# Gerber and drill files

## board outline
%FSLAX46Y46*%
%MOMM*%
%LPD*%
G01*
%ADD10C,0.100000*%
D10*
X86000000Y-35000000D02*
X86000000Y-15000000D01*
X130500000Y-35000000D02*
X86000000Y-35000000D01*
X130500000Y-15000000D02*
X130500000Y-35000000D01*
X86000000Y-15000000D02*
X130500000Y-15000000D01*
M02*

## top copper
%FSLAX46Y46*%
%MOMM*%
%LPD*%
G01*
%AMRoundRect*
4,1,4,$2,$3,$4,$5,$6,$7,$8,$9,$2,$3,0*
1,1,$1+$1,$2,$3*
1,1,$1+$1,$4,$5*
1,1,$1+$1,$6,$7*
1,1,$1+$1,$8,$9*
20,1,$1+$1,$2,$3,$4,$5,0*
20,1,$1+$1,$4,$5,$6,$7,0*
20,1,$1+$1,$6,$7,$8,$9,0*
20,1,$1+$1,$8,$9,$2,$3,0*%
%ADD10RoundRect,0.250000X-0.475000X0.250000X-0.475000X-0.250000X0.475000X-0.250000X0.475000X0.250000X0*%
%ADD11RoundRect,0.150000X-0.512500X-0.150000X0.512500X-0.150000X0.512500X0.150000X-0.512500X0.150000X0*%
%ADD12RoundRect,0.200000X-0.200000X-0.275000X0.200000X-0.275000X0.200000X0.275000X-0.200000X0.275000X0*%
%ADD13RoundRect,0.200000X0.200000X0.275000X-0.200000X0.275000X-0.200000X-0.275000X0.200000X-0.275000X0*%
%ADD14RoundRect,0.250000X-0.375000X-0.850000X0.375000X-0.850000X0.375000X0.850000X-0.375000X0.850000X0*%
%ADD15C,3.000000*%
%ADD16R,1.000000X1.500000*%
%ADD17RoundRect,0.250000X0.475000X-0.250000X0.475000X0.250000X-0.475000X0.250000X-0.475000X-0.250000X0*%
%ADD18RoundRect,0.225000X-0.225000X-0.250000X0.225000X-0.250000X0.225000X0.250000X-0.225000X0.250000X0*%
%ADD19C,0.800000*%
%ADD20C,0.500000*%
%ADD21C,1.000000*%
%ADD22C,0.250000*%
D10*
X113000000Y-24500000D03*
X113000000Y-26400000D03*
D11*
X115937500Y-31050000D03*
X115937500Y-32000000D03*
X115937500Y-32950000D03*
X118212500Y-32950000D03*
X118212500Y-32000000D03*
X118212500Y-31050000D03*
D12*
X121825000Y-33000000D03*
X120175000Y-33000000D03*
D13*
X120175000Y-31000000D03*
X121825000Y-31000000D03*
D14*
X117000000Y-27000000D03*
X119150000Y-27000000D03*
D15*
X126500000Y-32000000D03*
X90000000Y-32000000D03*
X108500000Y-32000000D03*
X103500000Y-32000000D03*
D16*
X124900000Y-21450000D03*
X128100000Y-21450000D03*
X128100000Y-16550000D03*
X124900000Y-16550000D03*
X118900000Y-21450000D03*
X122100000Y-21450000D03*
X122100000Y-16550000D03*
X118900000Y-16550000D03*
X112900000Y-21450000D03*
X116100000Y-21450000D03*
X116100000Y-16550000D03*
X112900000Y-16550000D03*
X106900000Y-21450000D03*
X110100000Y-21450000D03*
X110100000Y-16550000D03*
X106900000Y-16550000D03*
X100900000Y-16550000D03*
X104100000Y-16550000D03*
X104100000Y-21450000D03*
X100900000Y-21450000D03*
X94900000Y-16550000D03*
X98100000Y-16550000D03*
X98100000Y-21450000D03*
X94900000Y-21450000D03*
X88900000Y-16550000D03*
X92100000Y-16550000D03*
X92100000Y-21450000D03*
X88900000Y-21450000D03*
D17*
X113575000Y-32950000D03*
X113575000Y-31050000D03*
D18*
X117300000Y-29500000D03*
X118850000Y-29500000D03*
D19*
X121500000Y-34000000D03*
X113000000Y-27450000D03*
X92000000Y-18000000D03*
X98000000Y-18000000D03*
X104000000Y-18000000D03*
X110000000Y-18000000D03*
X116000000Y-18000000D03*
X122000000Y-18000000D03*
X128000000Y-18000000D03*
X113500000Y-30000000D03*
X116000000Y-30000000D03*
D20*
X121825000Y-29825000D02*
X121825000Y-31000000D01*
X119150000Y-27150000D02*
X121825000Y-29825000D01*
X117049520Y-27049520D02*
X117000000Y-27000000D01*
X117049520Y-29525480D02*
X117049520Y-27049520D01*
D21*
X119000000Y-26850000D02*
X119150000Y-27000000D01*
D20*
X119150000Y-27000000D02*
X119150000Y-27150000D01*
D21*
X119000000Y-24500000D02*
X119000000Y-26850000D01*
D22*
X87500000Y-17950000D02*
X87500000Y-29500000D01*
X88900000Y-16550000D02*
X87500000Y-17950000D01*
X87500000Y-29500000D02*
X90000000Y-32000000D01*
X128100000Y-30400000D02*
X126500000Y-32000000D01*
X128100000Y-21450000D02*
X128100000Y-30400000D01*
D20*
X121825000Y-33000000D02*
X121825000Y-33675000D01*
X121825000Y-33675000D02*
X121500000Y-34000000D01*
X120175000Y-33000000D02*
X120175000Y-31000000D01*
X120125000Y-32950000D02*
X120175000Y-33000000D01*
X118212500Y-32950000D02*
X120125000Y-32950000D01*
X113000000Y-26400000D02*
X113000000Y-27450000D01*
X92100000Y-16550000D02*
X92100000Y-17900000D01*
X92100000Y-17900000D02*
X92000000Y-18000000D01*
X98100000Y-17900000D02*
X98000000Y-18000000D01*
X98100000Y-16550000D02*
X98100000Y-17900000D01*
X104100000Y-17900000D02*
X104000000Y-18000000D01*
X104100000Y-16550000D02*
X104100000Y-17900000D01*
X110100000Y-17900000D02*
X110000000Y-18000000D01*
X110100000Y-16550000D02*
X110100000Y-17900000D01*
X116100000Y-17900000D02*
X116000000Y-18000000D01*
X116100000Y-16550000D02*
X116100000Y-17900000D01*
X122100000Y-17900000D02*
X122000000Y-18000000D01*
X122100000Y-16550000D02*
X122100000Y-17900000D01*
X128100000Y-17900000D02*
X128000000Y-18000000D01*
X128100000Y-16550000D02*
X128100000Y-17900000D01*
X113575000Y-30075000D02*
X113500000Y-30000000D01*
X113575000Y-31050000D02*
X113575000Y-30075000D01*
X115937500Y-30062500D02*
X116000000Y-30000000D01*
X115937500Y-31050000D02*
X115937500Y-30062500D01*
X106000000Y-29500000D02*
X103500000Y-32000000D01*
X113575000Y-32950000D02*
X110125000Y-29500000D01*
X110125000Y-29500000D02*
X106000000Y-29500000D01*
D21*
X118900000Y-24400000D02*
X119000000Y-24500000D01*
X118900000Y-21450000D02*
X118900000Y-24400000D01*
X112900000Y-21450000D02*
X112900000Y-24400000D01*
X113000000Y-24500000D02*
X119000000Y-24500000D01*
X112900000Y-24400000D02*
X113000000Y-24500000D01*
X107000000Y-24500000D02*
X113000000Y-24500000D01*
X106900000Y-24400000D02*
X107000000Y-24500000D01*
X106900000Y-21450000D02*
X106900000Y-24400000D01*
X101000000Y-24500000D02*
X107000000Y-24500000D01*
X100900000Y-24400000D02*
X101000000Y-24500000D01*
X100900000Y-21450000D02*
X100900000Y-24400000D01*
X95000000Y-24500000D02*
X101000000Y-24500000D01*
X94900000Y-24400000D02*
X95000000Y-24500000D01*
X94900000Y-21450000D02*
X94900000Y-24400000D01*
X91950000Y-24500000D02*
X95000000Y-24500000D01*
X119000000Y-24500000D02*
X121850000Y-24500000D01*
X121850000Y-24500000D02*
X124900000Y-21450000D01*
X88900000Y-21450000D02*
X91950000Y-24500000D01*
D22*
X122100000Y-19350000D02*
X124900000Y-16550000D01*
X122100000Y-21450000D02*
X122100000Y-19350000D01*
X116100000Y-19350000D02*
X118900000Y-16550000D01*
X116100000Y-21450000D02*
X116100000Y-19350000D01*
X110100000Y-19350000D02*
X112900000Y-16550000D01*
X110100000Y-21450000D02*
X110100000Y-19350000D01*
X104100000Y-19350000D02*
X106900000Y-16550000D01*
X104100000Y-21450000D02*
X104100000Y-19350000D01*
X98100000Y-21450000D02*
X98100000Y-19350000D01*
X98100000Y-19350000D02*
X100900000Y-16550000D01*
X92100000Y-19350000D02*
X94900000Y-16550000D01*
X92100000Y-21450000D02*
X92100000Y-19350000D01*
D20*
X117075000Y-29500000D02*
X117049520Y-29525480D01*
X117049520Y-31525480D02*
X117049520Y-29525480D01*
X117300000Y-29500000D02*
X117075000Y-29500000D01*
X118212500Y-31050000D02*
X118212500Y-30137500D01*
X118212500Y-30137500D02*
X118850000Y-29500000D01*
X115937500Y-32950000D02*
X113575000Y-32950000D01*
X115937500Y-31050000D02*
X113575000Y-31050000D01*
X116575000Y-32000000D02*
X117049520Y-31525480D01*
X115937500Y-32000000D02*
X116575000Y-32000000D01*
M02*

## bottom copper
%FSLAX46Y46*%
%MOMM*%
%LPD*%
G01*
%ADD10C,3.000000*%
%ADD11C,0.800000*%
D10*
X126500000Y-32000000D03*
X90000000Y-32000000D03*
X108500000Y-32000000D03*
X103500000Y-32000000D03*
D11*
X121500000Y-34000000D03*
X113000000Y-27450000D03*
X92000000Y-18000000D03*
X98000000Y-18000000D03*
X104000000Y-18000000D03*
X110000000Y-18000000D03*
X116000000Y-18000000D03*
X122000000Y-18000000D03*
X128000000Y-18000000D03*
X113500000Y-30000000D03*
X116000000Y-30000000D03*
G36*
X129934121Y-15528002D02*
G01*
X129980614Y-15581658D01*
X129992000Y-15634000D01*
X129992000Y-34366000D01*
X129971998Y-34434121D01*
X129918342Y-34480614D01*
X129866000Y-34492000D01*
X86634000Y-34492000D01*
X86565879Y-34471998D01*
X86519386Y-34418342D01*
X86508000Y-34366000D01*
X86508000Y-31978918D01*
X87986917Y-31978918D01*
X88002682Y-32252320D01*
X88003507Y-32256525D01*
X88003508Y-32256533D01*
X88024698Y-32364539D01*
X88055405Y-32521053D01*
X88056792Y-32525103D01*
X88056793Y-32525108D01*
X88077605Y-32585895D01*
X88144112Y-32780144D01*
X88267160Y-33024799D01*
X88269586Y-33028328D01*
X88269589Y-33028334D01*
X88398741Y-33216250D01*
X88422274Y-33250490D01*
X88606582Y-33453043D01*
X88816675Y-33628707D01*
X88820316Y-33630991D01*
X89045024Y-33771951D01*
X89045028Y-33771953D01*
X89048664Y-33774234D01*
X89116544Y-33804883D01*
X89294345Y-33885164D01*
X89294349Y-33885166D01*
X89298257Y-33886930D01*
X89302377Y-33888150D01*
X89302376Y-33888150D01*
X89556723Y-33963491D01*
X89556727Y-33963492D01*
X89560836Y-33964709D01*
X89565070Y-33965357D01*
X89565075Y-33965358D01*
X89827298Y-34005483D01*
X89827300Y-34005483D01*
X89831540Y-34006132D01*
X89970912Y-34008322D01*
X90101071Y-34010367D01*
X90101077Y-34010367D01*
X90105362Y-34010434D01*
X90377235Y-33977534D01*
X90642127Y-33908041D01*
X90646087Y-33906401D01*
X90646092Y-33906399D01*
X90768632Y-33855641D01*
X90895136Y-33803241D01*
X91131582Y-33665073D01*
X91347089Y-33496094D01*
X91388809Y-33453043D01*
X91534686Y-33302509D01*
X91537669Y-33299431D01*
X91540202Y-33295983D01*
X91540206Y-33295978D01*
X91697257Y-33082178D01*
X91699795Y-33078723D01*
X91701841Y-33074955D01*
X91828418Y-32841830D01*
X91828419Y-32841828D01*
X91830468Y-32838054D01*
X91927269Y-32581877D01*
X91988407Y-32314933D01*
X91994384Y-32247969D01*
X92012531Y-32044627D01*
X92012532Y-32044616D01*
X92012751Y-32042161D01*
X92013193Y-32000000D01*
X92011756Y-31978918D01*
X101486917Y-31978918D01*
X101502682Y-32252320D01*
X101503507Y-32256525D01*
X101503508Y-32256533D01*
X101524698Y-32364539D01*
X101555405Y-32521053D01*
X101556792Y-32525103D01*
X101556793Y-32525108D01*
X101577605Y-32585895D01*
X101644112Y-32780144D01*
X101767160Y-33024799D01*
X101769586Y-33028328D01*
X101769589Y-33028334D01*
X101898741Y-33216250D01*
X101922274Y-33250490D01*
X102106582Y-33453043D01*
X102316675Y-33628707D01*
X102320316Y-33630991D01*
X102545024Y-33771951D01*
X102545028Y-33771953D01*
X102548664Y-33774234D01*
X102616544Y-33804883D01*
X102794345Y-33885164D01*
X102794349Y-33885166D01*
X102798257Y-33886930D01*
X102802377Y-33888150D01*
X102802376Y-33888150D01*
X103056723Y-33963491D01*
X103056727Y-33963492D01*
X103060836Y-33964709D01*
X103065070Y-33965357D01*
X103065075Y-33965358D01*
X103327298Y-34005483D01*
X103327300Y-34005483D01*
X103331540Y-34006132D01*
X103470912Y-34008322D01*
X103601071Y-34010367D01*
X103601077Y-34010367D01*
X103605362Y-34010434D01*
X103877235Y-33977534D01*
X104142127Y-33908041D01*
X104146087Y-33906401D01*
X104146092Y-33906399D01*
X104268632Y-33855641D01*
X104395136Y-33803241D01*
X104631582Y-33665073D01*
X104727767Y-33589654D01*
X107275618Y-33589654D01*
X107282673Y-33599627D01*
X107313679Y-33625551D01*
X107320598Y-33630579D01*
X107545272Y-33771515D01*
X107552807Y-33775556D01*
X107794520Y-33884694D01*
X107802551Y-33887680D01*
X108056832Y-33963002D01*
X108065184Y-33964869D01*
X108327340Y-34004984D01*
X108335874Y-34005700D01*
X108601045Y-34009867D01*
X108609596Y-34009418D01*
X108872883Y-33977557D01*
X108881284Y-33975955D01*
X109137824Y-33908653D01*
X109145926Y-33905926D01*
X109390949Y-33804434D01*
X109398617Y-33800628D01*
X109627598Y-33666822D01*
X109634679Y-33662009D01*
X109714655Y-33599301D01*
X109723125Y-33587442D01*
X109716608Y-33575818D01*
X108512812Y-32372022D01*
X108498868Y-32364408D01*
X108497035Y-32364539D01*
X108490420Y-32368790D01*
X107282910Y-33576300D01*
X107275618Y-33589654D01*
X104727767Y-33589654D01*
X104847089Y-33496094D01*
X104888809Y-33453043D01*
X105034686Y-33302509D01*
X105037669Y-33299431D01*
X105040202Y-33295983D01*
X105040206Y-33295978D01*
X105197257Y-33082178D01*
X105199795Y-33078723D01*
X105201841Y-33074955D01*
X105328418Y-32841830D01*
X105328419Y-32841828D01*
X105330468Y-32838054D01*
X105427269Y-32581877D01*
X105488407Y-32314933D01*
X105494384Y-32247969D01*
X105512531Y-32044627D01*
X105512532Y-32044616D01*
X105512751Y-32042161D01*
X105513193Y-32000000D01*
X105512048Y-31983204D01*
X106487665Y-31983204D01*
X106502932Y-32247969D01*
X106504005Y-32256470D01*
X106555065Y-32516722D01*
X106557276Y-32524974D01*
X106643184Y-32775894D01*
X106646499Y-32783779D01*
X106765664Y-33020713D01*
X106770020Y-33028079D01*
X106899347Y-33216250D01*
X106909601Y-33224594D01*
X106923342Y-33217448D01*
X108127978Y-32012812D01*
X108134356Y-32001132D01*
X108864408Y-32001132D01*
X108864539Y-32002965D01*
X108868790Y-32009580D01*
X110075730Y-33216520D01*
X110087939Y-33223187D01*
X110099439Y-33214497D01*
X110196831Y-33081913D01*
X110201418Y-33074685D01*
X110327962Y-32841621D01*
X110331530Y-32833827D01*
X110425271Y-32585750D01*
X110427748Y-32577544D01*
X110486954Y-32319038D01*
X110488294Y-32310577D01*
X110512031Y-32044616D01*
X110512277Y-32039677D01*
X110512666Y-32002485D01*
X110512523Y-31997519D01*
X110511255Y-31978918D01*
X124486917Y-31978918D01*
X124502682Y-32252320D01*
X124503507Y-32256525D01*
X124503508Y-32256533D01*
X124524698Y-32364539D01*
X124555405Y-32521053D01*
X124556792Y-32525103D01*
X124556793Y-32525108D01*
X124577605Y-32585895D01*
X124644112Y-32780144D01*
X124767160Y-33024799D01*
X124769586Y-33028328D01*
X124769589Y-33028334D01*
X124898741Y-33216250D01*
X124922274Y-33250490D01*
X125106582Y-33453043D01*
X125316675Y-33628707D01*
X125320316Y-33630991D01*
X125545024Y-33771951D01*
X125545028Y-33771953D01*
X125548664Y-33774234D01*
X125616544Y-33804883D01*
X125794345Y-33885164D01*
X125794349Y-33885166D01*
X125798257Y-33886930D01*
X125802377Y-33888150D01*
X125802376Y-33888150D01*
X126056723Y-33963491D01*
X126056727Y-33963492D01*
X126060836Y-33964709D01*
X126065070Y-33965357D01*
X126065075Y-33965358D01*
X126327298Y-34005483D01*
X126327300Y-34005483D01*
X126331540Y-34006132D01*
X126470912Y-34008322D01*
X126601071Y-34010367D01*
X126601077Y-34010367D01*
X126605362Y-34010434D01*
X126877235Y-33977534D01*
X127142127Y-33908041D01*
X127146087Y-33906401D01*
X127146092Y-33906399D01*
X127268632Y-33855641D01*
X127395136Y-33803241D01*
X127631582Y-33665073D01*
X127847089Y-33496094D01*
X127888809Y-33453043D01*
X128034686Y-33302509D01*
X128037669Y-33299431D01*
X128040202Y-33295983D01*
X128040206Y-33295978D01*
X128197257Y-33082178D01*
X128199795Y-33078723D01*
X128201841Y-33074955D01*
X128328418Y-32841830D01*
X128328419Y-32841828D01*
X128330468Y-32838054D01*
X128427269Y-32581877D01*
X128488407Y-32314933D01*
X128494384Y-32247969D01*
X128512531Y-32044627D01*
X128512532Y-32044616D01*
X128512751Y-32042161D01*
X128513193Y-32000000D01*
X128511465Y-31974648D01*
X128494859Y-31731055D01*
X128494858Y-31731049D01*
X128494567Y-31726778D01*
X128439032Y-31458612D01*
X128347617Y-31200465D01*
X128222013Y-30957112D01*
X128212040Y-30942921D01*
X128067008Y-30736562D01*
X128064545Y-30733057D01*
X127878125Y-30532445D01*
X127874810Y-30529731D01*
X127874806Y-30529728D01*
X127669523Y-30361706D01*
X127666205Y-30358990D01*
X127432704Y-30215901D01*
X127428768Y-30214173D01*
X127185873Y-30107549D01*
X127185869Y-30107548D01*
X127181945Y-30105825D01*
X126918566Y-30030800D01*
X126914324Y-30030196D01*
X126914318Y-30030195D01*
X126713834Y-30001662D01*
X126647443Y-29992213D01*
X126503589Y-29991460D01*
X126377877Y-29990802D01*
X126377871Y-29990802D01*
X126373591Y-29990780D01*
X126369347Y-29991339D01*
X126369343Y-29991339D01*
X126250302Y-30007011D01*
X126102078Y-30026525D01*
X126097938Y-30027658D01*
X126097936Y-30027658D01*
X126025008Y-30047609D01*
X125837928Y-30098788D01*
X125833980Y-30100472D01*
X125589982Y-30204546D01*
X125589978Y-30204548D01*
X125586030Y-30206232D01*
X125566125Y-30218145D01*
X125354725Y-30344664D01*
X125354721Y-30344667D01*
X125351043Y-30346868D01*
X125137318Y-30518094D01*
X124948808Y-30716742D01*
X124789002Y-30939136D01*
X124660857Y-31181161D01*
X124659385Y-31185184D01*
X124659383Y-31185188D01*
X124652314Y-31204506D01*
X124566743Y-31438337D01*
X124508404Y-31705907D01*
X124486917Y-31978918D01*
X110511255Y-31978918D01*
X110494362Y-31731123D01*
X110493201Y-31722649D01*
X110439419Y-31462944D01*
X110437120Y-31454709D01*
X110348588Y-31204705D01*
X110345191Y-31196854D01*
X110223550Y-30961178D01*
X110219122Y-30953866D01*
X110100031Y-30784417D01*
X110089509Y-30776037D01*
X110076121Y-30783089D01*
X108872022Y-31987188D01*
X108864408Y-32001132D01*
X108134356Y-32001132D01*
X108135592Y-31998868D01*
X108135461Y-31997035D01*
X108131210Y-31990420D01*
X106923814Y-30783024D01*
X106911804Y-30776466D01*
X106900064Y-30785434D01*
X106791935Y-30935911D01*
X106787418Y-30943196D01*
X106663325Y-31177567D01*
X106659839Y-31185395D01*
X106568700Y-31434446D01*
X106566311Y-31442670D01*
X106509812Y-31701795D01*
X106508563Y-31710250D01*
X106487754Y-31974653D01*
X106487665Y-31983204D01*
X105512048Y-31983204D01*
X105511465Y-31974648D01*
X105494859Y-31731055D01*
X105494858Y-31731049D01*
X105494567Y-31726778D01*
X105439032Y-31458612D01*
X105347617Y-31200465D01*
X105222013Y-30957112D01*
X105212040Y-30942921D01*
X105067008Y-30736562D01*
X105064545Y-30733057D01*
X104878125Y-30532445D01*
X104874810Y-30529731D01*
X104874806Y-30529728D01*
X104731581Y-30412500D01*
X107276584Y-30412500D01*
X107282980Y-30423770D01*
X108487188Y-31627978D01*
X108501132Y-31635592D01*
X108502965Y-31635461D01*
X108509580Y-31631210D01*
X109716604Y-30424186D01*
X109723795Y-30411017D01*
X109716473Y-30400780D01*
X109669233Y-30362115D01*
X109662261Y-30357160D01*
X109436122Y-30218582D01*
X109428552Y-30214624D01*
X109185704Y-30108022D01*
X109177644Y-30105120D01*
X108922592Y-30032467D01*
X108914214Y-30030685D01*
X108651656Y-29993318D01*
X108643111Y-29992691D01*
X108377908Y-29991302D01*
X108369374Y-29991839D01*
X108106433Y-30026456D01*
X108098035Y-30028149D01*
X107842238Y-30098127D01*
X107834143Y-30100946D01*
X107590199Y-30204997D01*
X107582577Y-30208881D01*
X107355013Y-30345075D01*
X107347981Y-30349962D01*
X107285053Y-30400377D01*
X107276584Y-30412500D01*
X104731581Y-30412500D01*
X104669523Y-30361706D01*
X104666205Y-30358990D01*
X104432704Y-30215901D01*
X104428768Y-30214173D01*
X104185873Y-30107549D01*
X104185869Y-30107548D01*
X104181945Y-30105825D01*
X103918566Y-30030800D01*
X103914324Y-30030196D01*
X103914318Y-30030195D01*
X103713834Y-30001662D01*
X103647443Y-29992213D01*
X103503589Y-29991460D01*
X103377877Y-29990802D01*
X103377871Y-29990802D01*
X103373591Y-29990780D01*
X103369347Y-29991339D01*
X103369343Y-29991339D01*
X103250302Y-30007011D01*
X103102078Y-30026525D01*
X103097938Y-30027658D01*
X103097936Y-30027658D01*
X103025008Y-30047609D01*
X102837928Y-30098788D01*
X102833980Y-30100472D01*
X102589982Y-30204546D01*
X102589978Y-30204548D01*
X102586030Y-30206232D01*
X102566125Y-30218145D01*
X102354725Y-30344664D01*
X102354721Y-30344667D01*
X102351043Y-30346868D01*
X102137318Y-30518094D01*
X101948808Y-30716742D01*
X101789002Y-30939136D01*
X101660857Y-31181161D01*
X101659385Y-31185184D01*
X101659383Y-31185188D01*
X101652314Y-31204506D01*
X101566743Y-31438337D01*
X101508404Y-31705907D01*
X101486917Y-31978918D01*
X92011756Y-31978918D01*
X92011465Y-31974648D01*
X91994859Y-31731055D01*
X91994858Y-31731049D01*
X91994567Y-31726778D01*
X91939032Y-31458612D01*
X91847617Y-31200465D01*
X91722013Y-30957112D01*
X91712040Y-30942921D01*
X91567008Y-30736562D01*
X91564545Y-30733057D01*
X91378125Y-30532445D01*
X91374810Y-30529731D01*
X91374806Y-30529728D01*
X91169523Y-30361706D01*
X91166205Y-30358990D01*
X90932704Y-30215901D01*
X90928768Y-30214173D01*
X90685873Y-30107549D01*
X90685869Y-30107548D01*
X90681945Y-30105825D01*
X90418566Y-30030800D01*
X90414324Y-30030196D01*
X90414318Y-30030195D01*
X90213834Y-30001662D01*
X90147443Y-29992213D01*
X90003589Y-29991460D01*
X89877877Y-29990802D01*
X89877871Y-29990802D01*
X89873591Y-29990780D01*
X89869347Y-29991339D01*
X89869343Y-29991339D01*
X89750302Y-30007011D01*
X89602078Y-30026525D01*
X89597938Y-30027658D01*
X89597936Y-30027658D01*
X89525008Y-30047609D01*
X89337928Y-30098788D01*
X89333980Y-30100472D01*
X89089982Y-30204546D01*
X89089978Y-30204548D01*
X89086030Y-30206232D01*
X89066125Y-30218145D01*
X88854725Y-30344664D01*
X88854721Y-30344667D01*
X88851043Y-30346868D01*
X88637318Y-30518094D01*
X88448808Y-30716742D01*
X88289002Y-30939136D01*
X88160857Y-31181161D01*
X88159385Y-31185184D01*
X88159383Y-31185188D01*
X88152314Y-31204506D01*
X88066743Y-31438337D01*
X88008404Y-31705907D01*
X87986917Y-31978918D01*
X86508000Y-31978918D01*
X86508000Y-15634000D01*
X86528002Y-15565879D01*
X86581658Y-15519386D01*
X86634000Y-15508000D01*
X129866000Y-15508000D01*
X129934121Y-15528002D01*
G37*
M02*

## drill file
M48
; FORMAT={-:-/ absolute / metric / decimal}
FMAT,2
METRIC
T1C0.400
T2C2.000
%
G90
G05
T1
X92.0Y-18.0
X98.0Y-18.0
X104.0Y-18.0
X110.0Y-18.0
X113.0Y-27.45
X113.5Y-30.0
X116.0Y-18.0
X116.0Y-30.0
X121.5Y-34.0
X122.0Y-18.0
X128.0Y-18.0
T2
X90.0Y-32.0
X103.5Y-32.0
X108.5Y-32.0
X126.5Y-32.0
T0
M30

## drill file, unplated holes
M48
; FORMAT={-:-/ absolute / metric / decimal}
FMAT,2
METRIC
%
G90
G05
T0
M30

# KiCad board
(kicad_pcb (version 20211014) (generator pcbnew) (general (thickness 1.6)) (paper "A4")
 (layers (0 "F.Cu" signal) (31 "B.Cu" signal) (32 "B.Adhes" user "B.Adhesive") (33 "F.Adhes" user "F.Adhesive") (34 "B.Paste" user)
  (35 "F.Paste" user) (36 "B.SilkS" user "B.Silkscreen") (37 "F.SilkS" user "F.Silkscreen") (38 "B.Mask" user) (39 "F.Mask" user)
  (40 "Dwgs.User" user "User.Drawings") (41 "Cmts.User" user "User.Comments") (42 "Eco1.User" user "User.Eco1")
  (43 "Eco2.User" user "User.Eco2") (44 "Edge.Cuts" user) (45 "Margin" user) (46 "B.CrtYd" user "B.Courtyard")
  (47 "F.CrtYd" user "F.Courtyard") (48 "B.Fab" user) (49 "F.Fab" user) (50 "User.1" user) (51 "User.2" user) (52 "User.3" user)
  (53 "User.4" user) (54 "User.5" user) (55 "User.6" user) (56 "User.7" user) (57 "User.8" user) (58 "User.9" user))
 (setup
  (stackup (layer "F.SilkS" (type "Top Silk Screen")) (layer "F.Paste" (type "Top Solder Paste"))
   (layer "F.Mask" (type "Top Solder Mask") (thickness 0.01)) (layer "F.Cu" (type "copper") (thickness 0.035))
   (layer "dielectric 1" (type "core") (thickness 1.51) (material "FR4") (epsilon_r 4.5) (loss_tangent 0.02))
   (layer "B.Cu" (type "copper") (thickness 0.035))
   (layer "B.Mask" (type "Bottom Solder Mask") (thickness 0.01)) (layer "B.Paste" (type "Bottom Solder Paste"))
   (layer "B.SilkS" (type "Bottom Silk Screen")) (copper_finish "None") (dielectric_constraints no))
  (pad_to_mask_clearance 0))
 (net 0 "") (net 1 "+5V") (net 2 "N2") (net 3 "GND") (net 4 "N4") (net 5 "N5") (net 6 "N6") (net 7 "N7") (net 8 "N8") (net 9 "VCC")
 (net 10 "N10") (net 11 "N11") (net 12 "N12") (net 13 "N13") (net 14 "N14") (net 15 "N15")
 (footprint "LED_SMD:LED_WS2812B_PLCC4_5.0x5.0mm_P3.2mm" (layer "F.Cu") (at 114.5 19 90)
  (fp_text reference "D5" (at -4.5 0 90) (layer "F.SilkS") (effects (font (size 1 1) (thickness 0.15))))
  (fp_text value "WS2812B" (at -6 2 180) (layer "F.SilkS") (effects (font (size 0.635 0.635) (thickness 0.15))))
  (pad "1" smd rect (at -2.45 -1.6 90) (size 1.5 1) (layers "F.Cu" "F.Paste" "F.Mask") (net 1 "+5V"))
  (pad "2" smd rect (at -2.45 1.6 90) (size 1.5 1) (layers "F.Cu" "F.Paste" "F.Mask") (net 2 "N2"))
  (pad "3" smd rect (at 2.45 1.6 90) (size 1.5 1) (layers "F.Cu" "F.Paste" "F.Mask") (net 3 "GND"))
  (pad "4" smd rect (at 2.45 -1.6 90) (size 1.5 1) (layers "F.Cu" "F.Paste" "F.Mask") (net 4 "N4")))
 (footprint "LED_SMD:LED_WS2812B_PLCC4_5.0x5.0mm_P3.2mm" (layer "F.Cu") (at 90.5 19 90)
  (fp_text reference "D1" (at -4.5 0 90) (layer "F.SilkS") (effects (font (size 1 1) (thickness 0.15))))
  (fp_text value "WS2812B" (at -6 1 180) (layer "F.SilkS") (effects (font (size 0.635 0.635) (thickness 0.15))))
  (pad "1" smd rect (at -2.45 -1.6 90) (size 1.5 1) (layers "F.Cu" "F.Paste" "F.Mask") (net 1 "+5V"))
  (pad "2" smd rect (at -2.45 1.6 90) (size 1.5 1) (layers "F.Cu" "F.Paste" "F.Mask") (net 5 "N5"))
  (pad "3" smd rect (at 2.45 1.6 90) (size 1.5 1) (layers "F.Cu" "F.Paste" "F.Mask") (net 3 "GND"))
  (pad "4" smd rect (at 2.45 -1.6 90) (size 1.5 1) (layers "F.Cu" "F.Paste" "F.Mask") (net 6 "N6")))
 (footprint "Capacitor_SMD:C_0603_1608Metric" (layer "F.Cu") (at 118.075 29.5)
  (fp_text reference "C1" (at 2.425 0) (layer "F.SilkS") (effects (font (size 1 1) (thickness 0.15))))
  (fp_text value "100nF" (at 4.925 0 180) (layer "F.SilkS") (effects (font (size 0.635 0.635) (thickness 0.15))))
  (pad "1" smd roundrect (at -0.775 0) (size 0.9 0.95) (layers "F.Cu" "F.Paste" "F.Mask") (roundrect_rratio 0.25) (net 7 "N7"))
  (pad "2" smd roundrect (at 0.775 0) (size 0.9 0.95) (layers "F.Cu" "F.Paste" "F.Mask") (roundrect_rratio 0.25) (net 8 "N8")))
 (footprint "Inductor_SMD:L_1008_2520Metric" (layer "F.Cu") (at 118.075 27)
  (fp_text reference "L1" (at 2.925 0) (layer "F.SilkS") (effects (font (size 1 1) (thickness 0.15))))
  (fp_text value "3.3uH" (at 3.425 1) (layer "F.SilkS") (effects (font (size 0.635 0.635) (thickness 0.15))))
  (pad "1" smd roundrect (at -1.075 0) (size 1.25 2.2) (layers "F.Cu" "F.Paste" "F.Mask") (roundrect_rratio 0.2) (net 7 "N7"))
  (pad "2" smd roundrect (at 1.075 0) (size 1.25 2.2) (layers "F.Cu" "F.Paste" "F.Mask") (roundrect_rratio 0.2) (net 1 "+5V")))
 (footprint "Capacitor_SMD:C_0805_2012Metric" (layer "F.Cu") (at 113 25.45 -90)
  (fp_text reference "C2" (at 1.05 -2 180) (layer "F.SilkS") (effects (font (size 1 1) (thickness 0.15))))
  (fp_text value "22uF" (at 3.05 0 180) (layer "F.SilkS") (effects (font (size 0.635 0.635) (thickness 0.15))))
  (pad "1" smd roundrect (at -0.95 0 270) (size 1 1.45) (layers "F.Cu" "F.Paste" "F.Mask") (roundrect_rratio 0.25) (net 1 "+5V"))
  (pad "2" smd roundrect (at 0.95 0 270) (size 1 1.45) (layers "F.Cu" "F.Paste" "F.Mask") (roundrect_rratio 0.25) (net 3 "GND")))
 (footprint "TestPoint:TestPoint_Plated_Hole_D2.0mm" (layer "F.Cu") (at 90 32)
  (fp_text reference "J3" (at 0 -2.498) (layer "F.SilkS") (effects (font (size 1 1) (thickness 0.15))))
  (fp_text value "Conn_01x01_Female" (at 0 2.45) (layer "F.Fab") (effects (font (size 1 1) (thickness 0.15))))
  (pad "1" thru_hole circle (at 0 0) (size 3 3) (drill 2) (layers *.Cu *.Mask) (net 6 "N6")))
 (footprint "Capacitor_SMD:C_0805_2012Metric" (layer "F.Cu") (at 113.575 32 90)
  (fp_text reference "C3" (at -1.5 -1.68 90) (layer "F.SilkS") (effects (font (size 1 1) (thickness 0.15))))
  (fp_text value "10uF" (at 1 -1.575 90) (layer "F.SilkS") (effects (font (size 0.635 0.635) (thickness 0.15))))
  (pad "1" smd roundrect (at -0.95 0 90) (size 1 1.45) (layers "F.Cu" "F.Paste" "F.Mask") (roundrect_rratio 0.25) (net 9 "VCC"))
  (pad "2" smd roundrect (at 0.95 0 90) (size 1 1.45) (layers "F.Cu" "F.Paste" "F.Mask") (roundrect_rratio 0.25) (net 3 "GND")))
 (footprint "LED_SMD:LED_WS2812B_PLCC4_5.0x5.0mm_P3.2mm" (layer "F.Cu") (at 120.5 19 90)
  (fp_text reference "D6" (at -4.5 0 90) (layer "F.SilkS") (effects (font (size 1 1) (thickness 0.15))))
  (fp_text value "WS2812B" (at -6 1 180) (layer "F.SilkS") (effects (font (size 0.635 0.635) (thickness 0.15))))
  (pad "1" smd rect (at -2.45 -1.6 90) (size 1.5 1) (layers "F.Cu" "F.Paste" "F.Mask") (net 1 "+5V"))
  (pad "2" smd rect (at -2.45 1.6 90) (size 1.5 1) (layers "F.Cu" "F.Paste" "F.Mask") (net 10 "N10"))
  (pad "3" smd rect (at 2.45 1.6 90) (size 1.5 1) (layers "F.Cu" "F.Paste" "F.Mask") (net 3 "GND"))
  (pad "4" smd rect (at 2.45 -1.6 90) (size 1.5 1) (layers "F.Cu" "F.Paste" "F.Mask") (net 2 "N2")))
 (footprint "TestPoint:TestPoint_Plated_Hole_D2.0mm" (layer "F.Cu") (at 103.5 32)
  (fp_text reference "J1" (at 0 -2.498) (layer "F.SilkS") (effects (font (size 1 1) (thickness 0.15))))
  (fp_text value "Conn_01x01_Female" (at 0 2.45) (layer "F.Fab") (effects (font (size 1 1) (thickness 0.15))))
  (pad "1" thru_hole circle (at 0 0) (size 3 3) (drill 2) (layers *.Cu *.Mask) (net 9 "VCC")))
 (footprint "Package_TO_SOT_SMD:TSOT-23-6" (layer "F.Cu") (at 117.075 32)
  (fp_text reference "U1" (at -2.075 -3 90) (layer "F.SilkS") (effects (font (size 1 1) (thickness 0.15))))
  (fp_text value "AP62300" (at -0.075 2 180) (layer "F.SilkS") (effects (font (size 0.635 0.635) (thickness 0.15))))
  (pad "1" smd roundrect (at -1.1375 -0.95) (size 1.325 0.6) (layers "F.Cu" "F.Paste" "F.Mask") (roundrect_rratio 0.25) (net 3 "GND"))
  (pad "2" smd roundrect (at -1.1375 0) (size 1.325 0.6) (layers "F.Cu" "F.Paste" "F.Mask") (roundrect_rratio 0.25) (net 7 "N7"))
  (pad "3" smd roundrect (at -1.1375 0.95) (size 1.325 0.6) (layers "F.Cu" "F.Paste" "F.Mask") (roundrect_rratio 0.25) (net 9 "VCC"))
  (pad "4" smd roundrect (at 1.1375 0.95) (size 1.325 0.6) (layers "F.Cu" "F.Paste" "F.Mask") (roundrect_rratio 0.25) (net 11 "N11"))
  (pad "5" smd roundrect (at 1.1375 0) (size 1.325 0.6) (layers "F.Cu" "F.Paste" "F.Mask") (roundrect_rratio 0.25) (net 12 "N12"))
  (pad "6" smd roundrect (at 1.1375 -0.95) (size 1.325 0.6) (layers "F.Cu" "F.Paste" "F.Mask") (roundrect_rratio 0.25) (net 8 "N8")))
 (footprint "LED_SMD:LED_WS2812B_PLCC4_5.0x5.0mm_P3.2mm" (layer "F.Cu") (at 102.5 19 90)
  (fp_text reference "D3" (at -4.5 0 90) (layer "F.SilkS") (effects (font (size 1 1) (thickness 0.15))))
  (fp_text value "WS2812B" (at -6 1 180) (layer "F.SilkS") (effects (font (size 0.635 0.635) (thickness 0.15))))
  (pad "1" smd rect (at -2.45 -1.6 90) (size 1.5 1) (layers "F.Cu" "F.Paste" "F.Mask") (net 1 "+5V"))
  (pad "2" smd rect (at -2.45 1.6 90) (size 1.5 1) (layers "F.Cu" "F.Paste" "F.Mask") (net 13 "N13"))
  (pad "3" smd rect (at 2.45 1.6 90) (size 1.5 1) (layers "F.Cu" "F.Paste" "F.Mask") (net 3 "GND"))
  (pad "4" smd rect (at 2.45 -1.6 90) (size 1.5 1) (layers "F.Cu" "F.Paste" "F.Mask") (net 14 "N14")))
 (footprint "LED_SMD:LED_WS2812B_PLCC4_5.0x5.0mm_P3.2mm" (layer "F.Cu") (at 126.5 19 90)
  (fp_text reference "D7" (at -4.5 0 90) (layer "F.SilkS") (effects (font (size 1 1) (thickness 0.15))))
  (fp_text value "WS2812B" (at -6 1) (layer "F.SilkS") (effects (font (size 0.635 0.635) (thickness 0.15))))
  (pad "1" smd rect (at -2.45 -1.6 90) (size 1.5 1) (layers "F.Cu" "F.Paste" "F.Mask") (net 1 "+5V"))
  (pad "2" smd rect (at -2.45 1.6 90) (size 1.5 1) (layers "F.Cu" "F.Paste" "F.Mask") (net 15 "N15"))
  (pad "3" smd rect (at 2.45 1.6 90) (size 1.5 1) (layers "F.Cu" "F.Paste" "F.Mask") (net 3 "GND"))
  (pad "4" smd rect (at 2.45 -1.6 90) (size 1.5 1) (layers "F.Cu" "F.Paste" "F.Mask") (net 10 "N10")))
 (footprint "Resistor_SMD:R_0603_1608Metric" (layer "F.Cu") (at 121 31 180)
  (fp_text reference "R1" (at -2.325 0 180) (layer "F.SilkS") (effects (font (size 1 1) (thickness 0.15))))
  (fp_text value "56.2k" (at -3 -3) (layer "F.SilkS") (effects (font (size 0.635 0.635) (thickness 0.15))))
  (pad "1" smd roundrect (at -0.825 0 180) (size 0.8 0.95) (layers "F.Cu" "F.Paste" "F.Mask") (roundrect_rratio 0.25) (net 1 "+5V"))
  (pad "2" smd roundrect (at 0.825 0 180) (size 0.8 0.95) (layers "F.Cu" "F.Paste" "F.Mask") (roundrect_rratio 0.25) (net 11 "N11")))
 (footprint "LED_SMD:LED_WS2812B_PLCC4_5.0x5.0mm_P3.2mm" (layer "F.Cu") (at 96.5 19 90)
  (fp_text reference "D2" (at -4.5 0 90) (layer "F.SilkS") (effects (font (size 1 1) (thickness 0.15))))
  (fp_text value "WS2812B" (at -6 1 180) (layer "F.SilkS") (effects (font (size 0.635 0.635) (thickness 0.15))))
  (pad "1" smd rect (at -2.45 -1.6 90) (size 1.5 1) (layers "F.Cu" "F.Paste" "F.Mask") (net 1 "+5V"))
  (pad "2" smd rect (at -2.45 1.6 90) (size 1.5 1) (layers "F.Cu" "F.Paste" "F.Mask") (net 14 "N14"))
  (pad "3" smd rect (at 2.45 1.6 90) (size 1.5 1) (layers "F.Cu" "F.Paste" "F.Mask") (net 3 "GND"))
  (pad "4" smd rect (at 2.45 -1.6 90) (size 1.5 1) (layers "F.Cu" "F.Paste" "F.Mask") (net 5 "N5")))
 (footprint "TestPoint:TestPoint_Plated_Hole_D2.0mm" (layer "F.Cu") (at 126.5 32)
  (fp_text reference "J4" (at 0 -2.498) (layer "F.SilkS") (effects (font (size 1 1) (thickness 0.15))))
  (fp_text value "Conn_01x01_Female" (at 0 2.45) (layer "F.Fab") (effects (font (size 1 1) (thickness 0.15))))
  (pad "1" thru_hole circle (at 0 0) (size 3 3) (drill 2) (layers *.Cu *.Mask) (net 15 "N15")))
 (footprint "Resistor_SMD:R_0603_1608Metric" (layer "F.Cu") (at 121 33)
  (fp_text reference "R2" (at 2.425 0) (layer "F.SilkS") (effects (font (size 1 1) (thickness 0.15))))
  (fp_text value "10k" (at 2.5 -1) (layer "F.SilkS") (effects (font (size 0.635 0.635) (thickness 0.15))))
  (pad "1" smd roundrect (at -0.825 0) (size 0.8 0.95) (layers "F.Cu" "F.Paste" "F.Mask") (roundrect_rratio 0.25) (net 11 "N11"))
  (pad "2" smd roundrect (at 0.825 0) (size 0.8 0.95) (layers "F.Cu" "F.Paste" "F.Mask") (roundrect_rratio 0.25) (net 3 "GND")))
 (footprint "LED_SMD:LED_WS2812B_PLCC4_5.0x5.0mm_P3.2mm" (layer "F.Cu") (at 108.5 19 90)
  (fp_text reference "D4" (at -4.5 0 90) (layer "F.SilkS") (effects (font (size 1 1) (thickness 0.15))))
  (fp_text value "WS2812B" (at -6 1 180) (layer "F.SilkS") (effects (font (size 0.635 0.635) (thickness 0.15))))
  (pad "1" smd rect (at -2.45 -1.6 90) (size 1.5 1) (layers "F.Cu" "F.Paste" "F.Mask") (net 1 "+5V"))
  (pad "2" smd rect (at -2.45 1.6 90) (size 1.5 1) (layers "F.Cu" "F.Paste" "F.Mask") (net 4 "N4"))
  (pad "3" smd rect (at 2.45 1.6 90) (size 1.5 1) (layers "F.Cu" "F.Paste" "F.Mask") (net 3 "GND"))
  (pad "4" smd rect (at 2.45 -1.6 90) (size 1.5 1) (layers "F.Cu" "F.Paste" "F.Mask") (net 13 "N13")))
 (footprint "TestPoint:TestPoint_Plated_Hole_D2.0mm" (layer "F.Cu") (at 108.5 32)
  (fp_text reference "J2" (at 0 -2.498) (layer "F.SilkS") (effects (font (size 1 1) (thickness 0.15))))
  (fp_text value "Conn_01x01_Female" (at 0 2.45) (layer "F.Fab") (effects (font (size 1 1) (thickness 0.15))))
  (pad "1" thru_hole circle (at 0 0) (size 3 3) (drill 2) (layers *.Cu *.Mask) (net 3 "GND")))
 (gr_line (start 130.5 15) (end 130.5 35) (layer "Edge.Cuts") (width 0.1))
 (gr_line (start 130.5 35) (end 86 35) (layer "Edge.Cuts") (width 0.1))
 (gr_line (start 86 15) (end 130.5 15) (layer "Edge.Cuts") (width 0.1))
 (gr_line (start 86 35) (end 86 15) (layer "Edge.Cuts") (width 0.1))
 (segment (start 115.9375 32) (end 116.575 32) (width 0.5) (layer "F.Cu") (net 7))
 (segment (start 117.075 29.5) (end 117.04952 29.52548) (width 0.5) (layer "F.Cu") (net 7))
 (segment (start 117.3 29.5) (end 117.075 29.5) (width 0.5) (layer "F.Cu") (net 7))
 (segment (start 117.04952 31.52548) (end 117.04952 29.52548) (width 0.5) (layer "F.Cu") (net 7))
 (segment (start 116.575 32) (end 117.04952 31.52548) (width 0.5) (layer "F.Cu") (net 7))
 (segment (start 117.04952 27.04952) (end 117 27) (width 0.5) (layer "F.Cu") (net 7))
 (segment (start 117.04952 29.52548) (end 117.04952 27.04952) (width 0.5) (layer "F.Cu") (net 7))
 (segment (start 118.2125 30.1375) (end 118.85 29.5) (width 0.5) (layer "F.Cu") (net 8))
 (segment (start 118.2125 31.05) (end 118.2125 30.1375) (width 0.5) (layer "F.Cu") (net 8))
 (segment (start 88.9 21.45) (end 91.95 24.5) (width 1) (layer "F.Cu") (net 1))
 (segment (start 94.9 24.4) (end 95 24.5) (width 1) (layer "F.Cu") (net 1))
 (segment (start 119.15 27) (end 119.15 27.15) (width 0.5) (layer "F.Cu") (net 1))
 (segment (start 107 24.5) (end 113 24.5) (width 1) (layer "F.Cu") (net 1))
 (segment (start 118.9 21.45) (end 118.9 24.4) (width 1) (layer "F.Cu") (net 1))
 (segment (start 112.9 24.4) (end 113 24.5) (width 1) (layer "F.Cu") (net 1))
 (segment (start 119 24.5) (end 119 26.85) (width 1) (layer "F.Cu") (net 1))
 (segment (start 100.9 24.4) (end 101 24.5) (width 1) (layer "F.Cu") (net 1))
 (segment (start 113 24.5) (end 119 24.5) (width 1) (layer "F.Cu") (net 1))
 (segment (start 94.9 21.45) (end 94.9 24.4) (width 1) (layer "F.Cu") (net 1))
 (segment (start 119.15 27.15) (end 121.825 29.825) (width 0.5) (layer "F.Cu") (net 1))
 (segment (start 119 24.5) (end 121.85 24.5) (width 1) (layer "F.Cu") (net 1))
 (segment (start 118.9 24.4) (end 119 24.5) (width 1) (layer "F.Cu") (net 1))
 (segment (start 101 24.5) (end 107 24.5) (width 1) (layer "F.Cu") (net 1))
 (segment (start 91.95 24.5) (end 95 24.5) (width 1) (layer "F.Cu") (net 1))
 (segment (start 106.9 21.45) (end 106.9 24.4) (width 1) (layer "F.Cu") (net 1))
 (segment (start 106.9 24.4) (end 107 24.5) (width 1) (layer "F.Cu") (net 1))
 (segment (start 95 24.5) (end 101 24.5) (width 1) (layer "F.Cu") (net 1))
 (segment (start 112.9 21.45) (end 112.9 24.4) (width 1) (layer "F.Cu") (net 1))
 (segment (start 121.825 29.825) (end 121.825 31) (width 0.5) (layer "F.Cu") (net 1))
 (segment (start 119 26.85) (end 119.15 27) (width 1) (layer "F.Cu") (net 1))
 (segment (start 100.9 21.45) (end 100.9 24.4) (width 1) (layer "F.Cu") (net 1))
 (segment (start 121.85 24.5) (end 124.9 21.45) (width 1) (layer "F.Cu") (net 1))
 (segment (start 98.1 17.9) (end 98 18) (width 0.5) (layer "F.Cu") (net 3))
 (segment (start 92.1 17.9) (end 92 18) (width 0.5) (layer "F.Cu") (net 3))
 (segment (start 113 26.4) (end 113 27.45) (width 0.5) (layer "F.Cu") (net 3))
 (segment (start 121.825 33.675) (end 121.5 34) (width 0.5) (layer "F.Cu") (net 3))
 (segment (start 116.1 16.55) (end 116.1 17.9) (width 0.5) (layer "F.Cu") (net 3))
 (segment (start 128.1 17.9) (end 128 18) (width 0.5) (layer "F.Cu") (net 3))
 (segment (start 115.9375 31.05) (end 113.575 31.05) (width 0.5) (layer "F.Cu") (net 3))
 (segment (start 121.825 33) (end 121.825 33.675) (width 0.5) (layer "F.Cu") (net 3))
 (segment (start 115.9375 30.0625) (end 116 30) (width 0.5) (layer "F.Cu") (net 3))
 (segment (start 110.1 17.9) (end 110 18) (width 0.5) (layer "F.Cu") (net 3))
 (segment (start 104.1 17.9) (end 104 18) (width 0.5) (layer "F.Cu") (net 3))
 (segment (start 92.1 16.55) (end 92.1 17.9) (width 0.5) (layer "F.Cu") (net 3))
 (segment (start 122.1 17.9) (end 122 18) (width 0.5) (layer "F.Cu") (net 3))
 (segment (start 113.575 30.075) (end 113.5 30) (width 0.5) (layer "F.Cu") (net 3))
 (segment (start 128.1 16.55) (end 128.1 17.9) (width 0.5) (layer "F.Cu") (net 3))
 (segment (start 104.1 16.55) (end 104.1 17.9) (width 0.5) (layer "F.Cu") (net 3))
 (segment (start 122.1 16.55) (end 122.1 17.9) (width 0.5) (layer "F.Cu") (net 3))
 (segment (start 98.1 16.55) (end 98.1 17.9) (width 0.5) (layer "F.Cu") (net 3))
 (segment (start 110.1 16.55) (end 110.1 17.9) (width 0.5) (layer "F.Cu") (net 3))
 (segment (start 115.9375 31.05) (end 115.9375 30.0625) (width 0.5) (layer "F.Cu") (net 3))
 (segment (start 116.1 17.9) (end 116 18) (width 0.5) (layer "F.Cu") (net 3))
 (segment (start 113.575 31.05) (end 113.575 30.075) (width 0.5) (layer "F.Cu") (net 3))
 (via (at 92 18) (size 0.8) (drill 0.4) (layers "F.Cu" "B.Cu") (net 3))
 (via (at 116 18) (size 0.8) (drill 0.4) (layers "F.Cu" "B.Cu") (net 3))
 (via (at 122 18) (size 0.8) (drill 0.4) (layers "F.Cu" "B.Cu") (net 3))
 (via (at 104 18) (size 0.8) (drill 0.4) (layers "F.Cu" "B.Cu") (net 3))
 (via (at 121.5 34) (size 0.8) (drill 0.4) (layers "F.Cu" "B.Cu") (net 3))
 (via (at 98 18) (size 0.8) (drill 0.4) (layers "F.Cu" "B.Cu") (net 3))
 (via (at 110 18) (size 0.8) (drill 0.4) (layers "F.Cu" "B.Cu") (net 3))
 (via (at 113 27.45) (size 0.8) (drill 0.4) (layers "F.Cu" "B.Cu") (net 3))
 (via (at 113.5 30) (size 0.8) (drill 0.4) (layers "F.Cu" "B.Cu") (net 3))
 (via (at 116 30) (size 0.8) (drill 0.4) (layers "F.Cu" "B.Cu") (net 3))
 (via (at 128 18) (size 0.8) (drill 0.4) (layers "F.Cu" "B.Cu") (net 3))
 (segment (start 115.9375 32.95) (end 113.575 32.95) (width 0.5) (layer "F.Cu") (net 9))
 (segment (start 106 29.5) (end 103.5 32) (width 0.5) (layer "F.Cu") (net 9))
 (segment (start 113.575 32.95) (end 110.125 29.5) (width 0.5) (layer "F.Cu") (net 9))
 (segment (start 110.125 29.5) (end 106 29.5) (width 0.5) (layer "F.Cu") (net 9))
 (segment (start 92.1 21.45) (end 92.1 19.35) (width 0.25) (layer "F.Cu") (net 5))
 (segment (start 92.1 19.35) (end 94.9 16.55) (width 0.25) (layer "F.Cu") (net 5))
 (segment (start 88.9 16.55) (end 87.5 17.95) (width 0.25) (layer "F.Cu") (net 6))
 (segment (start 87.5 17.95) (end 87.5 29.5) (width 0.25) (layer "F.Cu") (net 6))
 (segment (start 87.5 29.5) (end 90 32) (width 0.25) (layer "F.Cu") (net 6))
 (segment (start 98.1 21.45) (end 98.1 19.35) (width 0.25) (layer "F.Cu") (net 14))
 (segment (start 98.1 19.35) (end 100.9 16.55) (width 0.25) (layer "F.Cu") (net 14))
 (segment (start 104.1 19.35) (end 106.9 16.55) (width 0.25) (layer "F.Cu") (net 13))
 (segment (start 104.1 21.45) (end 104.1 19.35) (width 0.25) (layer "F.Cu") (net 13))
 (segment (start 110.1 19.35) (end 112.9 16.55) (width 0.25) (layer "F.Cu") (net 4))
 (segment (start 110.1 21.45) (end 110.1 19.35) (width 0.25) (layer "F.Cu") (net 4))
 (segment (start 116.1 21.45) (end 116.1 19.35) (width 0.25) (layer "F.Cu") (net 2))
 (segment (start 116.1 19.35) (end 118.9 16.55) (width 0.25) (layer "F.Cu") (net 2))
 (segment (start 122.1 21.45) (end 122.1 19.35) (width 0.25) (layer "F.Cu") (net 10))
 (segment (start 122.1 19.35) (end 124.9 16.55) (width 0.25) (layer "F.Cu") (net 10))
 (segment (start 128.1 21.45) (end 128.1 30.4) (width 0.25) (layer "F.Cu") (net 15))
 (segment (start 128.1 30.4) (end 126.5 32) (width 0.25) (layer "F.Cu") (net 15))
 (segment (start 120.125 32.95) (end 120.175 33) (width 0.5) (layer "F.Cu") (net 11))
 (segment (start 118.2125 32.95) (end 120.125 32.95) (width 0.5) (layer "F.Cu") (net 11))
 (segment (start 120.175 33) (end 120.175 31) (width 0.5) (layer "F.Cu") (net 11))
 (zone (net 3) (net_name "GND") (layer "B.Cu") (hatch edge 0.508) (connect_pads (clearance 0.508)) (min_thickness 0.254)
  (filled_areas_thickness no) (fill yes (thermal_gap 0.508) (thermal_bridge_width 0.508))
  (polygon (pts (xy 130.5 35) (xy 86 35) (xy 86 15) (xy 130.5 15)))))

